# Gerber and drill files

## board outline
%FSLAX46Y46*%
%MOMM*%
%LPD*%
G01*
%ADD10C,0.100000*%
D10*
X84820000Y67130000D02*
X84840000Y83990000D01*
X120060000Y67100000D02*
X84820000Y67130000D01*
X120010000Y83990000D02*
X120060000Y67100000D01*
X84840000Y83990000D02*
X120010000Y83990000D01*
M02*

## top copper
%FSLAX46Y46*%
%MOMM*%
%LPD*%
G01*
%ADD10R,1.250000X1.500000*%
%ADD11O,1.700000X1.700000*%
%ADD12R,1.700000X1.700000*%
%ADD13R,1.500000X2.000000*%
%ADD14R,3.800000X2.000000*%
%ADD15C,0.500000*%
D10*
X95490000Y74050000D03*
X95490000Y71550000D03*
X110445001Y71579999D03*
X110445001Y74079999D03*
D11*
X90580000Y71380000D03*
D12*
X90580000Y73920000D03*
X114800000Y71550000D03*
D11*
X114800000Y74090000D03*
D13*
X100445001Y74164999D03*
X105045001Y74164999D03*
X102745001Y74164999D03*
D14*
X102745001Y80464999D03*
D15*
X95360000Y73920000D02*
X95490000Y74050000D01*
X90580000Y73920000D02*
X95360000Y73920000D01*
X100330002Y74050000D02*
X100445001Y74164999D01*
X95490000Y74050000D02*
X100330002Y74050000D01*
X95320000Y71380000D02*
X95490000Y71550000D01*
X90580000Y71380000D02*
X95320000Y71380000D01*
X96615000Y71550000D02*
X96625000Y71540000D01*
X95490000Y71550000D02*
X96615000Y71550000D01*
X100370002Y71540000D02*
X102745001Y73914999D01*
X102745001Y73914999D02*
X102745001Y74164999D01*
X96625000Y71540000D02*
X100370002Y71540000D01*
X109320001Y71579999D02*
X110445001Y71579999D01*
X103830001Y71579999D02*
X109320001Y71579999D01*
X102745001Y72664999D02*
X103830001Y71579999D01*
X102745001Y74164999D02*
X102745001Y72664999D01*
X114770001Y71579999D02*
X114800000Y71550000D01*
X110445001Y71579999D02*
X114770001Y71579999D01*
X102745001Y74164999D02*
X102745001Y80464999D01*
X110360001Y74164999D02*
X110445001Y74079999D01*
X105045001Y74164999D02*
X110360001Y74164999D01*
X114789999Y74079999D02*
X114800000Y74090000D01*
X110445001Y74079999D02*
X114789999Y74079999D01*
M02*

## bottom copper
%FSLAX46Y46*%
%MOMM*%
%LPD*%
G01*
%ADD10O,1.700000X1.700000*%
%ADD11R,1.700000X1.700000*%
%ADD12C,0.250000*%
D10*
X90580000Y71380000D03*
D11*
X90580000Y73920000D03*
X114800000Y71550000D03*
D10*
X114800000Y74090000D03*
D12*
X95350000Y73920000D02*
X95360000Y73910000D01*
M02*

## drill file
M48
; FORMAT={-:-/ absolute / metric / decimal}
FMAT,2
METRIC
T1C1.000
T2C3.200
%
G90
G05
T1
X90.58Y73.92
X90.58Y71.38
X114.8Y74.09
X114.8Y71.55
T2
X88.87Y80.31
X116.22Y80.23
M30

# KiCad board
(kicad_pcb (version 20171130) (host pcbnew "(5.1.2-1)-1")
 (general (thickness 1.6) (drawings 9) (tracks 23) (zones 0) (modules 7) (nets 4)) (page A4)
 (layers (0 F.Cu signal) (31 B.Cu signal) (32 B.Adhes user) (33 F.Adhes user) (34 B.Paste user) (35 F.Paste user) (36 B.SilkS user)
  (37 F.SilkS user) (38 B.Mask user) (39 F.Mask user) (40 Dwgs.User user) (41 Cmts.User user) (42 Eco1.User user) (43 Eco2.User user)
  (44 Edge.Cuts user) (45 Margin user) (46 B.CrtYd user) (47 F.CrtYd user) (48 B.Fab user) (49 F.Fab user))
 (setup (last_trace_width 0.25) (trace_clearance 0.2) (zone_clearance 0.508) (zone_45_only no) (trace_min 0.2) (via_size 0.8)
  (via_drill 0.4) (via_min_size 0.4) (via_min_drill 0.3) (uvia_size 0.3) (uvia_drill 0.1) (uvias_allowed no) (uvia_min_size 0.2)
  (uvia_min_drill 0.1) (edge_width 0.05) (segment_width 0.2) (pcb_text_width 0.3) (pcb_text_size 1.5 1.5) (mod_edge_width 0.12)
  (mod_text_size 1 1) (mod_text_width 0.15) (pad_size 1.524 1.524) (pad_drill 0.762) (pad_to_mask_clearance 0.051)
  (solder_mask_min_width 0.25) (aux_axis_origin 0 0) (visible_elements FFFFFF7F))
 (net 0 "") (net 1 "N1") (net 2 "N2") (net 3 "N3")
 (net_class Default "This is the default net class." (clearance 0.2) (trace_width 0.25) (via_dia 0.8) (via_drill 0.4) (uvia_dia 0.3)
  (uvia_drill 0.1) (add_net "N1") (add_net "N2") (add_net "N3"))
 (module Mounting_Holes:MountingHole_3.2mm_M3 (layer F.Cu) (at 116.22 -80.23)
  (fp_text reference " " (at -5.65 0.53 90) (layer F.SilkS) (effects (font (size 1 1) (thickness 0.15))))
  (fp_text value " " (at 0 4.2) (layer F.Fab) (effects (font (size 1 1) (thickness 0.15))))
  (pad 1 np_thru_hole circle (at 0 0) (size 3.2 3.2) (drill 3.2) (layers *.Cu *.Mask)))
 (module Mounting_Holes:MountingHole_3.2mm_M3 (layer F.Cu) (at 88.87 -80.31)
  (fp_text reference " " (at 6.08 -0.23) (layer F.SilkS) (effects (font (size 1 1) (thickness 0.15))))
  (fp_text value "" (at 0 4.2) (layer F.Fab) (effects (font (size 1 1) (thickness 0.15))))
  (pad 1 np_thru_hole circle (at 0 0) (size 3.2 3.2) (drill 3.2) (layers *.Cu *.Mask)))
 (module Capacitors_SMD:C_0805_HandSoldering (layer F.Cu) (at 95.49 -72.8 270)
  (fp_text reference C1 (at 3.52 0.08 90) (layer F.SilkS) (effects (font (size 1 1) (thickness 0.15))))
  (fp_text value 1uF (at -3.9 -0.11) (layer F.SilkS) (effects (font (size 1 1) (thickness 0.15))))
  (pad 1 smd rect (at -1.25 0 270) (size 1.5 1.25) (layers F.Cu F.Paste F.Mask) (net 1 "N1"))
  (pad 2 smd rect (at 1.25 0 270) (size 1.5 1.25) (layers F.Cu F.Paste F.Mask) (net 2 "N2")))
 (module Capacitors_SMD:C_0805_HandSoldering (layer F.Cu) (at 110.445001 -72.829999 270)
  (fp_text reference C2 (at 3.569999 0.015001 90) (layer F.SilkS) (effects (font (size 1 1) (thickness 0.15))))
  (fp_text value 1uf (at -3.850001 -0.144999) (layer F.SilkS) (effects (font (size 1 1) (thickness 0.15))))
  (pad 2 smd rect (at 1.25 0 270) (size 1.5 1.25) (layers F.Cu F.Paste F.Mask) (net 2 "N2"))
  (pad 1 smd rect (at -1.25 0 270) (size 1.5 1.25) (layers F.Cu F.Paste F.Mask) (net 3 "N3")))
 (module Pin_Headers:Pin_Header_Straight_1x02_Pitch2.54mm (layer F.Cu) (at 90.58 -73.92)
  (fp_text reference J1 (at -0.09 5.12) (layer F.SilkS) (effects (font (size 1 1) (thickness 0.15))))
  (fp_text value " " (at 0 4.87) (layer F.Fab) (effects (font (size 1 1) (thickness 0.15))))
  (pad 2 thru_hole oval (at 0 2.54) (size 1.7 1.7) (drill 1) (layers *.Cu *.Mask) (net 2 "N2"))
  (pad 1 thru_hole rect (at 0 0) (size 1.7 1.7) (drill 1) (layers *.Cu *.Mask) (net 1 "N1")))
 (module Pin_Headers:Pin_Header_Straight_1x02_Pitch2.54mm (layer F.Cu) (at 114.8 -71.55 180)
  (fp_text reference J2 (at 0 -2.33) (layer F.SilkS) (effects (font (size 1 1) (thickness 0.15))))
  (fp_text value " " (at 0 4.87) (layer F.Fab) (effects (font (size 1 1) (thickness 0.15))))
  (pad 1 thru_hole rect (at 0 0 180) (size 1.7 1.7) (drill 1) (layers *.Cu *.Mask) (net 2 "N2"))
  (pad 2 thru_hole oval (at 0 2.54 180) (size 1.7 1.7) (drill 1) (layers *.Cu *.Mask) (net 3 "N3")))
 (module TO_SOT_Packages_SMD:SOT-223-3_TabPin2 (layer F.Cu) (at 102.745001 -77.314999 90)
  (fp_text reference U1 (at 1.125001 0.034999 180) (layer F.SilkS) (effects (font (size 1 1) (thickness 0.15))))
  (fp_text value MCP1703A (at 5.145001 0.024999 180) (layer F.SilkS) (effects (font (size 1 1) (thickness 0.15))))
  (pad 1 smd rect (at -3.15 -2.3 90) (size 2 1.5) (layers F.Cu F.Paste F.Mask) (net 1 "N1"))
  (pad 3 smd rect (at -3.15 2.3 90) (size 2 1.5) (layers F.Cu F.Paste F.Mask) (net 3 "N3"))
  (pad 2 smd rect (at -3.15 0 90) (size 2 1.5) (layers F.Cu F.Paste F.Mask) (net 2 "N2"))
  (pad 2 smd rect (at 3.15 0 90) (size 2 3.8) (layers F.Cu F.Paste F.Mask) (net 2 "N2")))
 (gr_line (start 84.82 -67.13) (end 84.84 -83.99) (layer Edge.Cuts) (width 0.1))
 (gr_line (start 120.06 -67.1) (end 84.82 -67.13) (layer Edge.Cuts) (width 0.1))
 (gr_line (start 120.01 -83.99) (end 120.06 -67.1) (layer Edge.Cuts) (width 0.1))
 (gr_line (start 84.84 -83.99) (end 120.01 -83.99) (layer Edge.Cuts) (width 0.1))
 (segment (start 95.35 -73.92) (end 95.36 -73.91) (width 0.25) (layer B.Cu) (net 1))
 (segment (start 95.36 -73.92) (end 95.49 -74.05) (width 0.5) (layer F.Cu) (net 1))
 (segment (start 90.58 -73.92) (end 95.36 -73.92) (width 0.5) (layer F.Cu) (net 1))
 (segment (start 100.330002 -74.05) (end 100.445001 -74.164999) (width 0.5) (layer F.Cu) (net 1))
 (segment (start 95.49 -74.05) (end 100.330002 -74.05) (width 0.5) (layer F.Cu) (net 1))
 (segment (start 95.32 -71.38) (end 95.49 -71.55) (width 0.5) (layer F.Cu) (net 2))
 (segment (start 90.58 -71.38) (end 95.32 -71.38) (width 0.5) (layer F.Cu) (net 2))
 (segment (start 96.615 -71.55) (end 96.625 -71.54) (width 0.5) (layer F.Cu) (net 2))
 (segment (start 95.49 -71.55) (end 96.615 -71.55) (width 0.5) (layer F.Cu) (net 2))
 (segment (start 100.370002 -71.54) (end 102.745001 -73.914999) (width 0.5) (layer F.Cu) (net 2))
 (segment (start 102.745001 -73.914999) (end 102.745001 -74.164999) (width 0.5) (layer F.Cu) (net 2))
 (segment (start 96.625 -71.54) (end 100.370002 -71.54) (width 0.5) (layer F.Cu) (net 2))
 (segment (start 109.320001 -71.579999) (end 110.445001 -71.579999) (width 0.5) (layer F.Cu) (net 2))
 (segment (start 103.830001 -71.579999) (end 109.320001 -71.579999) (width 0.5) (layer F.Cu) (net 2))
 (segment (start 102.745001 -72.664999) (end 103.830001 -71.579999) (width 0.5) (layer F.Cu) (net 2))
 (segment (start 102.745001 -74.164999) (end 102.745001 -72.664999) (width 0.5) (layer F.Cu) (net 2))
 (segment (start 114.770001 -71.579999) (end 114.8 -71.55) (width 0.5) (layer F.Cu) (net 2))
 (segment (start 110.445001 -71.579999) (end 114.770001 -71.579999) (width 0.5) (layer F.Cu) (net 2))
 (segment (start 102.745001 -74.164999) (end 102.745001 -80.464999) (width 0.5) (layer F.Cu) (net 2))
 (segment (start 110.360001 -74.164999) (end 110.445001 -74.079999) (width 0.5) (layer F.Cu) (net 3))
 (segment (start 105.045001 -74.164999) (end 110.360001 -74.164999) (width 0.5) (layer F.Cu) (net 3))
 (segment (start 114.789999 -74.079999) (end 114.8 -74.09) (width 0.5) (layer F.Cu) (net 3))
 (segment (start 110.445001 -74.079999) (end 114.789999 -74.079999) (width 0.5) (layer F.Cu) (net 3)))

